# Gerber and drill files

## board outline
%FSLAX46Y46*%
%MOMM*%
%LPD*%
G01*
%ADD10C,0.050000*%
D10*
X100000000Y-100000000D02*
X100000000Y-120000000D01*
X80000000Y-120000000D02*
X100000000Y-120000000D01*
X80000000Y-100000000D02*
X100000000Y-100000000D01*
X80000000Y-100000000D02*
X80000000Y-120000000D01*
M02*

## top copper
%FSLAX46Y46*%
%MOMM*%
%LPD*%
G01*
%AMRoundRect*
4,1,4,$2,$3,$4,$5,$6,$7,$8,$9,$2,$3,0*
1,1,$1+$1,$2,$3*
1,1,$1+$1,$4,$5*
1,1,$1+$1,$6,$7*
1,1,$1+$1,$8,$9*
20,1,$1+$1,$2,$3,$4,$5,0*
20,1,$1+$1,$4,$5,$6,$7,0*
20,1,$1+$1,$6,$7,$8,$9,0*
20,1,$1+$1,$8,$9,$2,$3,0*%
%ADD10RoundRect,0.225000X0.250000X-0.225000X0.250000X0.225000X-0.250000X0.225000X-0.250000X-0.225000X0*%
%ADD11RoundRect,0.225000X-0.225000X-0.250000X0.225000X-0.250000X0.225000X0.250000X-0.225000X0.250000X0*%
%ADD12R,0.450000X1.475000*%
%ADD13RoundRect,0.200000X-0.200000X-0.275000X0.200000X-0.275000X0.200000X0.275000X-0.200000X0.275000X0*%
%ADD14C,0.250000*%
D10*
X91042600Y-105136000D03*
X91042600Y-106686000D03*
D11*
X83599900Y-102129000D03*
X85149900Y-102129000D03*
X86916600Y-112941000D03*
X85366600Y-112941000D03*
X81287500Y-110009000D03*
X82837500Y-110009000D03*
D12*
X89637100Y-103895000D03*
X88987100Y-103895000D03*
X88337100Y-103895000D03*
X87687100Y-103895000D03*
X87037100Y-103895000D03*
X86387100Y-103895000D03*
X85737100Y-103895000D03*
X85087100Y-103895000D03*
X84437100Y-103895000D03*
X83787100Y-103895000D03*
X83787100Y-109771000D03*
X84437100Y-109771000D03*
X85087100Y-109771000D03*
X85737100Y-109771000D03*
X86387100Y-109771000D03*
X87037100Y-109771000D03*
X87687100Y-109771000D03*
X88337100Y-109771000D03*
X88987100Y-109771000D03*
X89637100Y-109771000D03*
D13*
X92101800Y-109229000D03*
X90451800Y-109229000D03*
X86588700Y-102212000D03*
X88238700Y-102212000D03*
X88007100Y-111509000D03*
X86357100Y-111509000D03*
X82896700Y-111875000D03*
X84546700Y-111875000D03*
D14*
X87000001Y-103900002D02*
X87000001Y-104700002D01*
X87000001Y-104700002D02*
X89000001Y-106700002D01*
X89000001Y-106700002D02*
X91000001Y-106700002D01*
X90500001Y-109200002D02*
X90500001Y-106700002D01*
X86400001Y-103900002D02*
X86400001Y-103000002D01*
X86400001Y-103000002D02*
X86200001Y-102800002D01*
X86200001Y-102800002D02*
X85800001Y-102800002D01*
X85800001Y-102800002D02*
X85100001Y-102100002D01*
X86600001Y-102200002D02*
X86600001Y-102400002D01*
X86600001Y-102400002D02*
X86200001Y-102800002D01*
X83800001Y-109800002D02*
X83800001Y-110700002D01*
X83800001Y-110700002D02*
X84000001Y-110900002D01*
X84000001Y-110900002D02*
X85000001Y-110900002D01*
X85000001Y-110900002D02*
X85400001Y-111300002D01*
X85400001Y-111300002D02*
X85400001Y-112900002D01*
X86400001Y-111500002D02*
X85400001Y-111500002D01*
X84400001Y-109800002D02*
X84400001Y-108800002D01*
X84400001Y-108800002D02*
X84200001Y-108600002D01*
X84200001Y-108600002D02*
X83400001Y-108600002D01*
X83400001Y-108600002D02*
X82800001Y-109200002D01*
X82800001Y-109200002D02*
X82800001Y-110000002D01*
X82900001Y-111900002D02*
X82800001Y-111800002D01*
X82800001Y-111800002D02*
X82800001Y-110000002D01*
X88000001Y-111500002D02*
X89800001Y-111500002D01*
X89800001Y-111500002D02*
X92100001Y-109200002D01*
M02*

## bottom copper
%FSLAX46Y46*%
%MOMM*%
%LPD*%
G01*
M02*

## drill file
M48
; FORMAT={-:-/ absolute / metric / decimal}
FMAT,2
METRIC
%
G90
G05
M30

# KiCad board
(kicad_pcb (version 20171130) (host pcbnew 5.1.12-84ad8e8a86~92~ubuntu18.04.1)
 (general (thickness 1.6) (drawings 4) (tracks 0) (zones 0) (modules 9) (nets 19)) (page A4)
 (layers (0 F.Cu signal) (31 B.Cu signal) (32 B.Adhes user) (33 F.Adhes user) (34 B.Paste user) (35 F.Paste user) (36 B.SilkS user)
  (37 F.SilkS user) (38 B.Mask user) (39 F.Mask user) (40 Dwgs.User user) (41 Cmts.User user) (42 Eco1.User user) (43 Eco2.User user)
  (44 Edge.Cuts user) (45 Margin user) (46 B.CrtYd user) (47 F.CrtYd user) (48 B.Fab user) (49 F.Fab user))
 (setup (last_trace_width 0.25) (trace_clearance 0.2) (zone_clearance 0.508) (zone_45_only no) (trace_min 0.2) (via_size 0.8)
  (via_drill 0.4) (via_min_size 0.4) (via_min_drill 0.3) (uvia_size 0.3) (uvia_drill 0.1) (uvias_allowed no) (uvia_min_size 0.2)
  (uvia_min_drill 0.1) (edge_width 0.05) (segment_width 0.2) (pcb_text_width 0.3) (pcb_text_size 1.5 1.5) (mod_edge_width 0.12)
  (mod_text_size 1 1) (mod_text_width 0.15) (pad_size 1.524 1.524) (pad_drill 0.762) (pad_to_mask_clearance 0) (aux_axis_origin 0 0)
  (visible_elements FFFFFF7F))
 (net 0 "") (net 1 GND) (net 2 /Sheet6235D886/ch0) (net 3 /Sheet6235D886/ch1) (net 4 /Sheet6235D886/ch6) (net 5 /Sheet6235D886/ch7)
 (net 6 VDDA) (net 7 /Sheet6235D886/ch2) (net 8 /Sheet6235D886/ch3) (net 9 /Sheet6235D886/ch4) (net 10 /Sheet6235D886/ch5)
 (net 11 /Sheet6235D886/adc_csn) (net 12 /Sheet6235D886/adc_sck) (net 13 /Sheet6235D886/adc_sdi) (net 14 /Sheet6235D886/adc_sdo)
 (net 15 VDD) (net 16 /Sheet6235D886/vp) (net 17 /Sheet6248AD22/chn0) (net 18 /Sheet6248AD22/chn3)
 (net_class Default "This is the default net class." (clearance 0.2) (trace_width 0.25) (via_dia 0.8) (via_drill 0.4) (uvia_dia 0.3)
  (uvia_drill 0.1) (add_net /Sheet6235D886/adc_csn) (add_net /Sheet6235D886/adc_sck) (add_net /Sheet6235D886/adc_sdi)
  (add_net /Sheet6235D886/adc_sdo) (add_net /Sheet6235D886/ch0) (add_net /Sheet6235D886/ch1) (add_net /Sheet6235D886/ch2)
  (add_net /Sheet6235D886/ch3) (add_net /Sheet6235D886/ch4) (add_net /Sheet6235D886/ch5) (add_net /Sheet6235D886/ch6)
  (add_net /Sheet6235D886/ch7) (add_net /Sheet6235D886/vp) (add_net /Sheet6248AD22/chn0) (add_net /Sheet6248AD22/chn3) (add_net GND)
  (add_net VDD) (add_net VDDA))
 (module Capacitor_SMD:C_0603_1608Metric (layer F.Cu) (at 91.042600 105.911000 90.000000)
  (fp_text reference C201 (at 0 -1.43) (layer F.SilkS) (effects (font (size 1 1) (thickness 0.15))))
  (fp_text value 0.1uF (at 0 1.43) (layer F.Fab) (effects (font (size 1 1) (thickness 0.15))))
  (pad 2 smd roundrect (at 0.775 0 90.000000) (size 0.9 0.95) (layers F.Cu F.Mask F.Paste) (roundrect_rratio 0.25) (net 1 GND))
  (pad 1 smd roundrect (at -0.775 0 90.000000) (size 0.9 0.95) (layers F.Cu F.Mask F.Paste) (roundrect_rratio 0.25)
   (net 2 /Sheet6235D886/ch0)))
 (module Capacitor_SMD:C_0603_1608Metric (layer F.Cu) (at 84.374900 102.129000)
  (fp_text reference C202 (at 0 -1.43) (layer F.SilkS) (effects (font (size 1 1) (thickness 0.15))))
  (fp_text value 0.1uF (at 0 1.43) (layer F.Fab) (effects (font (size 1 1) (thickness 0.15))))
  (pad 1 smd roundrect (at -0.775 0) (size 0.9 0.95) (layers F.Cu F.Mask F.Paste) (roundrect_rratio 0.25) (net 1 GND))
  (pad 2 smd roundrect (at 0.775 0) (size 0.9 0.95) (layers F.Cu F.Mask F.Paste) (roundrect_rratio 0.25) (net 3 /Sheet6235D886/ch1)))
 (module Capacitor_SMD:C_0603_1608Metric (layer F.Cu) (at 86.141600 112.941000)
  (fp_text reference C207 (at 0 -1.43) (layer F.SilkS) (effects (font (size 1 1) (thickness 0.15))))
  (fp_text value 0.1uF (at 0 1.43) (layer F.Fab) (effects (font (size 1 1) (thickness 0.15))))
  (pad 2 smd roundrect (at 0.775 0) (size 0.9 0.95) (layers F.Cu F.Mask F.Paste) (roundrect_rratio 0.25) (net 1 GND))
  (pad 1 smd roundrect (at -0.775 0) (size 0.9 0.95) (layers F.Cu F.Mask F.Paste) (roundrect_rratio 0.25) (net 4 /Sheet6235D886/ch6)))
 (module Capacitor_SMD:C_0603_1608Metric (layer F.Cu) (at 82.062500 110.009000)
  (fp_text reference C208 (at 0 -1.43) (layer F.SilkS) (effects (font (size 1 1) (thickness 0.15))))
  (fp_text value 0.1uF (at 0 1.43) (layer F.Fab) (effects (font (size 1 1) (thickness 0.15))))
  (pad 1 smd roundrect (at -0.775 0) (size 0.9 0.95) (layers F.Cu F.Mask F.Paste) (roundrect_rratio 0.25) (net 1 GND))
  (pad 2 smd roundrect (at 0.775 0) (size 0.9 0.95) (layers F.Cu F.Mask F.Paste) (roundrect_rratio 0.25) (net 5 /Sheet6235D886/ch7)))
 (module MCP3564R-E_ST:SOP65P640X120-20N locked (layer F.Cu) (at 86.712100 106.833000 270.000000)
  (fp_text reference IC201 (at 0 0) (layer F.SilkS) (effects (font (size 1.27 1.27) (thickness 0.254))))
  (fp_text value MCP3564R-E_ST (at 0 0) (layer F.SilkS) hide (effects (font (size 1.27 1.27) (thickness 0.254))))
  (pad 1 smd rect (at -2.938 -2.925) (size 0.45 1.475) (layers F.Cu F.Mask F.Paste) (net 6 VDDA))
  (pad 2 smd rect (at -2.938 -2.275) (size 0.45 1.475) (layers F.Cu F.Mask F.Paste) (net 1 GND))
  (pad 3 smd rect (at -2.938 -1.625) (size 0.45 1.475) (layers F.Cu F.Mask F.Paste) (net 1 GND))
  (pad 4 smd rect (at -2.938 -0.975) (size 0.45 1.475) (layers F.Cu F.Mask F.Paste))
  (pad 5 smd rect (at -2.938 -0.325) (size 0.45 1.475) (layers F.Cu F.Mask F.Paste) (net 2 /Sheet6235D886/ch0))
  (pad 6 smd rect (at -2.938 0.325) (size 0.45 1.475) (layers F.Cu F.Mask F.Paste) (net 3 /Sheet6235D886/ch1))
  (pad 7 smd rect (at -2.938 0.975) (size 0.45 1.475) (layers F.Cu F.Mask F.Paste) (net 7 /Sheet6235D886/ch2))
  (pad 8 smd rect (at -2.938 1.625) (size 0.45 1.475) (layers F.Cu F.Mask F.Paste) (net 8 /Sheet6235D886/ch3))
  (pad 9 smd rect (at -2.938 2.275) (size 0.45 1.475) (layers F.Cu F.Mask F.Paste) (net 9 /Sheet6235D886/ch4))
  (pad 10 smd rect (at -2.938 2.925) (size 0.45 1.475) (layers F.Cu F.Mask F.Paste) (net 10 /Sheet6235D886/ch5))
  (pad 11 smd rect (at 2.938 2.925) (size 0.45 1.475) (layers F.Cu F.Mask F.Paste) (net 4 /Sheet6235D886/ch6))
  (pad 12 smd rect (at 2.938 2.275) (size 0.45 1.475) (layers F.Cu F.Mask F.Paste) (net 5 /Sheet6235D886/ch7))
  (pad 13 smd rect (at 2.938 1.625) (size 0.45 1.475) (layers F.Cu F.Mask F.Paste) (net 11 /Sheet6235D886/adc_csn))
  (pad 14 smd rect (at 2.938 0.975) (size 0.45 1.475) (layers F.Cu F.Mask F.Paste) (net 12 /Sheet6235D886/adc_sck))
  (pad 15 smd rect (at 2.938 0.325) (size 0.45 1.475) (layers F.Cu F.Mask F.Paste) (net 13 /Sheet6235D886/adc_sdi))
  (pad 16 smd rect (at 2.938 -0.325) (size 0.45 1.475) (layers F.Cu F.Mask F.Paste) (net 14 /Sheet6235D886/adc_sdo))
  (pad 17 smd rect (at 2.938 -0.975) (size 0.45 1.475) (layers F.Cu F.Mask F.Paste))
  (pad 18 smd rect (at 2.938 -1.625) (size 0.45 1.475) (layers F.Cu F.Mask F.Paste))
  (pad 19 smd rect (at 2.938 -2.275) (size 0.45 1.475) (layers F.Cu F.Mask F.Paste) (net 1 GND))
  (pad 20 smd rect (at 2.938 -2.925) (size 0.45 1.475) (layers F.Cu F.Mask F.Paste) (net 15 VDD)))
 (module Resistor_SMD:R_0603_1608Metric (layer F.Cu) (at 91.276800 109.229000)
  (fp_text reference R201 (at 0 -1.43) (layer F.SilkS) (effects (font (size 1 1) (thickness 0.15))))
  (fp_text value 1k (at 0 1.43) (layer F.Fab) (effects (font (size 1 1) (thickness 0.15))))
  (pad 2 smd roundrect (at 0.825 0) (size 0.8 0.95) (layers F.Cu F.Mask F.Paste) (roundrect_rratio 0.25) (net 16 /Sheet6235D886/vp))
  (pad 1 smd roundrect (at -0.825 0) (size 0.8 0.95) (layers F.Cu F.Mask F.Paste) (roundrect_rratio 0.25) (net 2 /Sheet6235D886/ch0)))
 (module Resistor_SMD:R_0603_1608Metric (layer F.Cu) (at 87.413700 102.212000)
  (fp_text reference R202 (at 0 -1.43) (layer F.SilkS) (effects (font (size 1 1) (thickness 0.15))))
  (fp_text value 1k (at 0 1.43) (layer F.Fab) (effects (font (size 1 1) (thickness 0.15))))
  (pad 1 smd roundrect (at -0.825 0) (size 0.8 0.95) (layers F.Cu F.Mask F.Paste) (roundrect_rratio 0.25) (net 3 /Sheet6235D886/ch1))
  (pad 2 smd roundrect (at 0.825 0) (size 0.8 0.95) (layers F.Cu F.Mask F.Paste) (roundrect_rratio 0.25) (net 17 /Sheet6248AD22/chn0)))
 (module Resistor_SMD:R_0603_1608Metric (layer F.Cu) (at 87.182100 111.509000)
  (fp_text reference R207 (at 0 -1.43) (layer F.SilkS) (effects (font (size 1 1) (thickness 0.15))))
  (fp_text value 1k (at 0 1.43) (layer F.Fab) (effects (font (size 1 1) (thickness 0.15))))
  (pad 2 smd roundrect (at 0.825 0) (size 0.8 0.95) (layers F.Cu F.Mask F.Paste) (roundrect_rratio 0.25) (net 16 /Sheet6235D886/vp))
  (pad 1 smd roundrect (at -0.825 0) (size 0.8 0.95) (layers F.Cu F.Mask F.Paste) (roundrect_rratio 0.25) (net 4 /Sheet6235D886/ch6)))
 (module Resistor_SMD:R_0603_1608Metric (layer F.Cu) (at 83.721700 111.875000)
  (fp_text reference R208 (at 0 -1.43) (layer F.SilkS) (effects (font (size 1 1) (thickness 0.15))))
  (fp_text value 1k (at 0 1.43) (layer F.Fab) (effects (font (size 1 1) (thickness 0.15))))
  (pad 1 smd roundrect (at -0.825 0) (size 0.8 0.95) (layers F.Cu F.Mask F.Paste) (roundrect_rratio 0.25) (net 5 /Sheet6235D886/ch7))
  (pad 2 smd roundrect (at 0.825 0) (size 0.8 0.95) (layers F.Cu F.Mask F.Paste) (roundrect_rratio 0.25) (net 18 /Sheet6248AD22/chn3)))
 (gr_line (start 100 100) (end 100 120) (layer Edge.Cuts) (width 0.05))
 (gr_line (start 80 120) (end 100 120) (layer Edge.Cuts) (width 0.05))
 (gr_line (start 80 100) (end 100 100) (layer Edge.Cuts) (width 0.05))
 (gr_line (start 80 100) (end 80 120) (layer Edge.Cuts) (width 0.05))
 (segment (start 87.000001 103.900002) (end 87.000001 104.700002) (width 0.250000) (layer F.Cu) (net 2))
 (segment (start 87.000001 104.700002) (end 89.000001 106.700002) (width 0.250000) (layer F.Cu) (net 2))
 (segment (start 89.000001 106.700002) (end 91.000001 106.700002) (width 0.250000) (layer F.Cu) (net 2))
 (segment (start 90.500001 109.200002) (end 90.500001 106.700002) (width 0.250000) (layer F.Cu) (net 2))
 (segment (start 86.400001 103.900002) (end 86.400001 103.000002) (width 0.250000) (layer F.Cu) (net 3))
 (segment (start 86.400001 103.000002) (end 86.200001 102.800002) (width 0.250000) (layer F.Cu) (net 3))
 (segment (start 86.200001 102.800002) (end 85.800001 102.800002) (width 0.250000) (layer F.Cu) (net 3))
 (segment (start 85.800001 102.800002) (end 85.100001 102.100002) (width 0.250000) (layer F.Cu) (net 3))
 (segment (start 86.600001 102.200002) (end 86.600001 102.400002) (width 0.250000) (layer F.Cu) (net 3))
 (segment (start 86.600001 102.400002) (end 86.200001 102.800002) (width 0.250000) (layer F.Cu) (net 3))
 (segment (start 83.800001 109.800002) (end 83.800001 110.700002) (width 0.250000) (layer F.Cu) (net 4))
 (segment (start 83.800001 110.700002) (end 84.000001 110.900002) (width 0.250000) (layer F.Cu) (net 4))
 (segment (start 84.000001 110.900002) (end 85.000001 110.900002) (width 0.250000) (layer F.Cu) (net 4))
 (segment (start 85.000001 110.900002) (end 85.400001 111.300002) (width 0.250000) (layer F.Cu) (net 4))
 (segment (start 85.400001 111.300002) (end 85.400001 112.900002) (width 0.250000) (layer F.Cu) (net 4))
 (segment (start 86.400001 111.500002) (end 85.400001 111.500002) (width 0.250000) (layer F.Cu) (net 4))
 (segment (start 84.400001 109.800002) (end 84.400001 108.800002) (width 0.250000) (layer F.Cu) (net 5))
 (segment (start 84.400001 108.800002) (end 84.200001 108.600002) (width 0.250000) (layer F.Cu) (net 5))
 (segment (start 84.200001 108.600002) (end 83.400001 108.600002) (width 0.250000) (layer F.Cu) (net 5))
 (segment (start 83.400001 108.600002) (end 82.800001 109.200002) (width 0.250000) (layer F.Cu) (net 5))
 (segment (start 82.800001 109.200002) (end 82.800001 110.000002) (width 0.250000) (layer F.Cu) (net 5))
 (segment (start 82.900001 111.900002) (end 82.800001 111.800002) (width 0.250000) (layer F.Cu) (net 5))
 (segment (start 82.800001 111.800002) (end 82.800001 110.000002) (width 0.250000) (layer F.Cu) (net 5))
 (segment (start 88.000001 111.500002) (end 89.800001 111.500002) (width 0.250000) (layer F.Cu) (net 16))
 (segment (start 89.800001 111.500002) (end 92.100001 109.200002) (width 0.250000) (layer F.Cu) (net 16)))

